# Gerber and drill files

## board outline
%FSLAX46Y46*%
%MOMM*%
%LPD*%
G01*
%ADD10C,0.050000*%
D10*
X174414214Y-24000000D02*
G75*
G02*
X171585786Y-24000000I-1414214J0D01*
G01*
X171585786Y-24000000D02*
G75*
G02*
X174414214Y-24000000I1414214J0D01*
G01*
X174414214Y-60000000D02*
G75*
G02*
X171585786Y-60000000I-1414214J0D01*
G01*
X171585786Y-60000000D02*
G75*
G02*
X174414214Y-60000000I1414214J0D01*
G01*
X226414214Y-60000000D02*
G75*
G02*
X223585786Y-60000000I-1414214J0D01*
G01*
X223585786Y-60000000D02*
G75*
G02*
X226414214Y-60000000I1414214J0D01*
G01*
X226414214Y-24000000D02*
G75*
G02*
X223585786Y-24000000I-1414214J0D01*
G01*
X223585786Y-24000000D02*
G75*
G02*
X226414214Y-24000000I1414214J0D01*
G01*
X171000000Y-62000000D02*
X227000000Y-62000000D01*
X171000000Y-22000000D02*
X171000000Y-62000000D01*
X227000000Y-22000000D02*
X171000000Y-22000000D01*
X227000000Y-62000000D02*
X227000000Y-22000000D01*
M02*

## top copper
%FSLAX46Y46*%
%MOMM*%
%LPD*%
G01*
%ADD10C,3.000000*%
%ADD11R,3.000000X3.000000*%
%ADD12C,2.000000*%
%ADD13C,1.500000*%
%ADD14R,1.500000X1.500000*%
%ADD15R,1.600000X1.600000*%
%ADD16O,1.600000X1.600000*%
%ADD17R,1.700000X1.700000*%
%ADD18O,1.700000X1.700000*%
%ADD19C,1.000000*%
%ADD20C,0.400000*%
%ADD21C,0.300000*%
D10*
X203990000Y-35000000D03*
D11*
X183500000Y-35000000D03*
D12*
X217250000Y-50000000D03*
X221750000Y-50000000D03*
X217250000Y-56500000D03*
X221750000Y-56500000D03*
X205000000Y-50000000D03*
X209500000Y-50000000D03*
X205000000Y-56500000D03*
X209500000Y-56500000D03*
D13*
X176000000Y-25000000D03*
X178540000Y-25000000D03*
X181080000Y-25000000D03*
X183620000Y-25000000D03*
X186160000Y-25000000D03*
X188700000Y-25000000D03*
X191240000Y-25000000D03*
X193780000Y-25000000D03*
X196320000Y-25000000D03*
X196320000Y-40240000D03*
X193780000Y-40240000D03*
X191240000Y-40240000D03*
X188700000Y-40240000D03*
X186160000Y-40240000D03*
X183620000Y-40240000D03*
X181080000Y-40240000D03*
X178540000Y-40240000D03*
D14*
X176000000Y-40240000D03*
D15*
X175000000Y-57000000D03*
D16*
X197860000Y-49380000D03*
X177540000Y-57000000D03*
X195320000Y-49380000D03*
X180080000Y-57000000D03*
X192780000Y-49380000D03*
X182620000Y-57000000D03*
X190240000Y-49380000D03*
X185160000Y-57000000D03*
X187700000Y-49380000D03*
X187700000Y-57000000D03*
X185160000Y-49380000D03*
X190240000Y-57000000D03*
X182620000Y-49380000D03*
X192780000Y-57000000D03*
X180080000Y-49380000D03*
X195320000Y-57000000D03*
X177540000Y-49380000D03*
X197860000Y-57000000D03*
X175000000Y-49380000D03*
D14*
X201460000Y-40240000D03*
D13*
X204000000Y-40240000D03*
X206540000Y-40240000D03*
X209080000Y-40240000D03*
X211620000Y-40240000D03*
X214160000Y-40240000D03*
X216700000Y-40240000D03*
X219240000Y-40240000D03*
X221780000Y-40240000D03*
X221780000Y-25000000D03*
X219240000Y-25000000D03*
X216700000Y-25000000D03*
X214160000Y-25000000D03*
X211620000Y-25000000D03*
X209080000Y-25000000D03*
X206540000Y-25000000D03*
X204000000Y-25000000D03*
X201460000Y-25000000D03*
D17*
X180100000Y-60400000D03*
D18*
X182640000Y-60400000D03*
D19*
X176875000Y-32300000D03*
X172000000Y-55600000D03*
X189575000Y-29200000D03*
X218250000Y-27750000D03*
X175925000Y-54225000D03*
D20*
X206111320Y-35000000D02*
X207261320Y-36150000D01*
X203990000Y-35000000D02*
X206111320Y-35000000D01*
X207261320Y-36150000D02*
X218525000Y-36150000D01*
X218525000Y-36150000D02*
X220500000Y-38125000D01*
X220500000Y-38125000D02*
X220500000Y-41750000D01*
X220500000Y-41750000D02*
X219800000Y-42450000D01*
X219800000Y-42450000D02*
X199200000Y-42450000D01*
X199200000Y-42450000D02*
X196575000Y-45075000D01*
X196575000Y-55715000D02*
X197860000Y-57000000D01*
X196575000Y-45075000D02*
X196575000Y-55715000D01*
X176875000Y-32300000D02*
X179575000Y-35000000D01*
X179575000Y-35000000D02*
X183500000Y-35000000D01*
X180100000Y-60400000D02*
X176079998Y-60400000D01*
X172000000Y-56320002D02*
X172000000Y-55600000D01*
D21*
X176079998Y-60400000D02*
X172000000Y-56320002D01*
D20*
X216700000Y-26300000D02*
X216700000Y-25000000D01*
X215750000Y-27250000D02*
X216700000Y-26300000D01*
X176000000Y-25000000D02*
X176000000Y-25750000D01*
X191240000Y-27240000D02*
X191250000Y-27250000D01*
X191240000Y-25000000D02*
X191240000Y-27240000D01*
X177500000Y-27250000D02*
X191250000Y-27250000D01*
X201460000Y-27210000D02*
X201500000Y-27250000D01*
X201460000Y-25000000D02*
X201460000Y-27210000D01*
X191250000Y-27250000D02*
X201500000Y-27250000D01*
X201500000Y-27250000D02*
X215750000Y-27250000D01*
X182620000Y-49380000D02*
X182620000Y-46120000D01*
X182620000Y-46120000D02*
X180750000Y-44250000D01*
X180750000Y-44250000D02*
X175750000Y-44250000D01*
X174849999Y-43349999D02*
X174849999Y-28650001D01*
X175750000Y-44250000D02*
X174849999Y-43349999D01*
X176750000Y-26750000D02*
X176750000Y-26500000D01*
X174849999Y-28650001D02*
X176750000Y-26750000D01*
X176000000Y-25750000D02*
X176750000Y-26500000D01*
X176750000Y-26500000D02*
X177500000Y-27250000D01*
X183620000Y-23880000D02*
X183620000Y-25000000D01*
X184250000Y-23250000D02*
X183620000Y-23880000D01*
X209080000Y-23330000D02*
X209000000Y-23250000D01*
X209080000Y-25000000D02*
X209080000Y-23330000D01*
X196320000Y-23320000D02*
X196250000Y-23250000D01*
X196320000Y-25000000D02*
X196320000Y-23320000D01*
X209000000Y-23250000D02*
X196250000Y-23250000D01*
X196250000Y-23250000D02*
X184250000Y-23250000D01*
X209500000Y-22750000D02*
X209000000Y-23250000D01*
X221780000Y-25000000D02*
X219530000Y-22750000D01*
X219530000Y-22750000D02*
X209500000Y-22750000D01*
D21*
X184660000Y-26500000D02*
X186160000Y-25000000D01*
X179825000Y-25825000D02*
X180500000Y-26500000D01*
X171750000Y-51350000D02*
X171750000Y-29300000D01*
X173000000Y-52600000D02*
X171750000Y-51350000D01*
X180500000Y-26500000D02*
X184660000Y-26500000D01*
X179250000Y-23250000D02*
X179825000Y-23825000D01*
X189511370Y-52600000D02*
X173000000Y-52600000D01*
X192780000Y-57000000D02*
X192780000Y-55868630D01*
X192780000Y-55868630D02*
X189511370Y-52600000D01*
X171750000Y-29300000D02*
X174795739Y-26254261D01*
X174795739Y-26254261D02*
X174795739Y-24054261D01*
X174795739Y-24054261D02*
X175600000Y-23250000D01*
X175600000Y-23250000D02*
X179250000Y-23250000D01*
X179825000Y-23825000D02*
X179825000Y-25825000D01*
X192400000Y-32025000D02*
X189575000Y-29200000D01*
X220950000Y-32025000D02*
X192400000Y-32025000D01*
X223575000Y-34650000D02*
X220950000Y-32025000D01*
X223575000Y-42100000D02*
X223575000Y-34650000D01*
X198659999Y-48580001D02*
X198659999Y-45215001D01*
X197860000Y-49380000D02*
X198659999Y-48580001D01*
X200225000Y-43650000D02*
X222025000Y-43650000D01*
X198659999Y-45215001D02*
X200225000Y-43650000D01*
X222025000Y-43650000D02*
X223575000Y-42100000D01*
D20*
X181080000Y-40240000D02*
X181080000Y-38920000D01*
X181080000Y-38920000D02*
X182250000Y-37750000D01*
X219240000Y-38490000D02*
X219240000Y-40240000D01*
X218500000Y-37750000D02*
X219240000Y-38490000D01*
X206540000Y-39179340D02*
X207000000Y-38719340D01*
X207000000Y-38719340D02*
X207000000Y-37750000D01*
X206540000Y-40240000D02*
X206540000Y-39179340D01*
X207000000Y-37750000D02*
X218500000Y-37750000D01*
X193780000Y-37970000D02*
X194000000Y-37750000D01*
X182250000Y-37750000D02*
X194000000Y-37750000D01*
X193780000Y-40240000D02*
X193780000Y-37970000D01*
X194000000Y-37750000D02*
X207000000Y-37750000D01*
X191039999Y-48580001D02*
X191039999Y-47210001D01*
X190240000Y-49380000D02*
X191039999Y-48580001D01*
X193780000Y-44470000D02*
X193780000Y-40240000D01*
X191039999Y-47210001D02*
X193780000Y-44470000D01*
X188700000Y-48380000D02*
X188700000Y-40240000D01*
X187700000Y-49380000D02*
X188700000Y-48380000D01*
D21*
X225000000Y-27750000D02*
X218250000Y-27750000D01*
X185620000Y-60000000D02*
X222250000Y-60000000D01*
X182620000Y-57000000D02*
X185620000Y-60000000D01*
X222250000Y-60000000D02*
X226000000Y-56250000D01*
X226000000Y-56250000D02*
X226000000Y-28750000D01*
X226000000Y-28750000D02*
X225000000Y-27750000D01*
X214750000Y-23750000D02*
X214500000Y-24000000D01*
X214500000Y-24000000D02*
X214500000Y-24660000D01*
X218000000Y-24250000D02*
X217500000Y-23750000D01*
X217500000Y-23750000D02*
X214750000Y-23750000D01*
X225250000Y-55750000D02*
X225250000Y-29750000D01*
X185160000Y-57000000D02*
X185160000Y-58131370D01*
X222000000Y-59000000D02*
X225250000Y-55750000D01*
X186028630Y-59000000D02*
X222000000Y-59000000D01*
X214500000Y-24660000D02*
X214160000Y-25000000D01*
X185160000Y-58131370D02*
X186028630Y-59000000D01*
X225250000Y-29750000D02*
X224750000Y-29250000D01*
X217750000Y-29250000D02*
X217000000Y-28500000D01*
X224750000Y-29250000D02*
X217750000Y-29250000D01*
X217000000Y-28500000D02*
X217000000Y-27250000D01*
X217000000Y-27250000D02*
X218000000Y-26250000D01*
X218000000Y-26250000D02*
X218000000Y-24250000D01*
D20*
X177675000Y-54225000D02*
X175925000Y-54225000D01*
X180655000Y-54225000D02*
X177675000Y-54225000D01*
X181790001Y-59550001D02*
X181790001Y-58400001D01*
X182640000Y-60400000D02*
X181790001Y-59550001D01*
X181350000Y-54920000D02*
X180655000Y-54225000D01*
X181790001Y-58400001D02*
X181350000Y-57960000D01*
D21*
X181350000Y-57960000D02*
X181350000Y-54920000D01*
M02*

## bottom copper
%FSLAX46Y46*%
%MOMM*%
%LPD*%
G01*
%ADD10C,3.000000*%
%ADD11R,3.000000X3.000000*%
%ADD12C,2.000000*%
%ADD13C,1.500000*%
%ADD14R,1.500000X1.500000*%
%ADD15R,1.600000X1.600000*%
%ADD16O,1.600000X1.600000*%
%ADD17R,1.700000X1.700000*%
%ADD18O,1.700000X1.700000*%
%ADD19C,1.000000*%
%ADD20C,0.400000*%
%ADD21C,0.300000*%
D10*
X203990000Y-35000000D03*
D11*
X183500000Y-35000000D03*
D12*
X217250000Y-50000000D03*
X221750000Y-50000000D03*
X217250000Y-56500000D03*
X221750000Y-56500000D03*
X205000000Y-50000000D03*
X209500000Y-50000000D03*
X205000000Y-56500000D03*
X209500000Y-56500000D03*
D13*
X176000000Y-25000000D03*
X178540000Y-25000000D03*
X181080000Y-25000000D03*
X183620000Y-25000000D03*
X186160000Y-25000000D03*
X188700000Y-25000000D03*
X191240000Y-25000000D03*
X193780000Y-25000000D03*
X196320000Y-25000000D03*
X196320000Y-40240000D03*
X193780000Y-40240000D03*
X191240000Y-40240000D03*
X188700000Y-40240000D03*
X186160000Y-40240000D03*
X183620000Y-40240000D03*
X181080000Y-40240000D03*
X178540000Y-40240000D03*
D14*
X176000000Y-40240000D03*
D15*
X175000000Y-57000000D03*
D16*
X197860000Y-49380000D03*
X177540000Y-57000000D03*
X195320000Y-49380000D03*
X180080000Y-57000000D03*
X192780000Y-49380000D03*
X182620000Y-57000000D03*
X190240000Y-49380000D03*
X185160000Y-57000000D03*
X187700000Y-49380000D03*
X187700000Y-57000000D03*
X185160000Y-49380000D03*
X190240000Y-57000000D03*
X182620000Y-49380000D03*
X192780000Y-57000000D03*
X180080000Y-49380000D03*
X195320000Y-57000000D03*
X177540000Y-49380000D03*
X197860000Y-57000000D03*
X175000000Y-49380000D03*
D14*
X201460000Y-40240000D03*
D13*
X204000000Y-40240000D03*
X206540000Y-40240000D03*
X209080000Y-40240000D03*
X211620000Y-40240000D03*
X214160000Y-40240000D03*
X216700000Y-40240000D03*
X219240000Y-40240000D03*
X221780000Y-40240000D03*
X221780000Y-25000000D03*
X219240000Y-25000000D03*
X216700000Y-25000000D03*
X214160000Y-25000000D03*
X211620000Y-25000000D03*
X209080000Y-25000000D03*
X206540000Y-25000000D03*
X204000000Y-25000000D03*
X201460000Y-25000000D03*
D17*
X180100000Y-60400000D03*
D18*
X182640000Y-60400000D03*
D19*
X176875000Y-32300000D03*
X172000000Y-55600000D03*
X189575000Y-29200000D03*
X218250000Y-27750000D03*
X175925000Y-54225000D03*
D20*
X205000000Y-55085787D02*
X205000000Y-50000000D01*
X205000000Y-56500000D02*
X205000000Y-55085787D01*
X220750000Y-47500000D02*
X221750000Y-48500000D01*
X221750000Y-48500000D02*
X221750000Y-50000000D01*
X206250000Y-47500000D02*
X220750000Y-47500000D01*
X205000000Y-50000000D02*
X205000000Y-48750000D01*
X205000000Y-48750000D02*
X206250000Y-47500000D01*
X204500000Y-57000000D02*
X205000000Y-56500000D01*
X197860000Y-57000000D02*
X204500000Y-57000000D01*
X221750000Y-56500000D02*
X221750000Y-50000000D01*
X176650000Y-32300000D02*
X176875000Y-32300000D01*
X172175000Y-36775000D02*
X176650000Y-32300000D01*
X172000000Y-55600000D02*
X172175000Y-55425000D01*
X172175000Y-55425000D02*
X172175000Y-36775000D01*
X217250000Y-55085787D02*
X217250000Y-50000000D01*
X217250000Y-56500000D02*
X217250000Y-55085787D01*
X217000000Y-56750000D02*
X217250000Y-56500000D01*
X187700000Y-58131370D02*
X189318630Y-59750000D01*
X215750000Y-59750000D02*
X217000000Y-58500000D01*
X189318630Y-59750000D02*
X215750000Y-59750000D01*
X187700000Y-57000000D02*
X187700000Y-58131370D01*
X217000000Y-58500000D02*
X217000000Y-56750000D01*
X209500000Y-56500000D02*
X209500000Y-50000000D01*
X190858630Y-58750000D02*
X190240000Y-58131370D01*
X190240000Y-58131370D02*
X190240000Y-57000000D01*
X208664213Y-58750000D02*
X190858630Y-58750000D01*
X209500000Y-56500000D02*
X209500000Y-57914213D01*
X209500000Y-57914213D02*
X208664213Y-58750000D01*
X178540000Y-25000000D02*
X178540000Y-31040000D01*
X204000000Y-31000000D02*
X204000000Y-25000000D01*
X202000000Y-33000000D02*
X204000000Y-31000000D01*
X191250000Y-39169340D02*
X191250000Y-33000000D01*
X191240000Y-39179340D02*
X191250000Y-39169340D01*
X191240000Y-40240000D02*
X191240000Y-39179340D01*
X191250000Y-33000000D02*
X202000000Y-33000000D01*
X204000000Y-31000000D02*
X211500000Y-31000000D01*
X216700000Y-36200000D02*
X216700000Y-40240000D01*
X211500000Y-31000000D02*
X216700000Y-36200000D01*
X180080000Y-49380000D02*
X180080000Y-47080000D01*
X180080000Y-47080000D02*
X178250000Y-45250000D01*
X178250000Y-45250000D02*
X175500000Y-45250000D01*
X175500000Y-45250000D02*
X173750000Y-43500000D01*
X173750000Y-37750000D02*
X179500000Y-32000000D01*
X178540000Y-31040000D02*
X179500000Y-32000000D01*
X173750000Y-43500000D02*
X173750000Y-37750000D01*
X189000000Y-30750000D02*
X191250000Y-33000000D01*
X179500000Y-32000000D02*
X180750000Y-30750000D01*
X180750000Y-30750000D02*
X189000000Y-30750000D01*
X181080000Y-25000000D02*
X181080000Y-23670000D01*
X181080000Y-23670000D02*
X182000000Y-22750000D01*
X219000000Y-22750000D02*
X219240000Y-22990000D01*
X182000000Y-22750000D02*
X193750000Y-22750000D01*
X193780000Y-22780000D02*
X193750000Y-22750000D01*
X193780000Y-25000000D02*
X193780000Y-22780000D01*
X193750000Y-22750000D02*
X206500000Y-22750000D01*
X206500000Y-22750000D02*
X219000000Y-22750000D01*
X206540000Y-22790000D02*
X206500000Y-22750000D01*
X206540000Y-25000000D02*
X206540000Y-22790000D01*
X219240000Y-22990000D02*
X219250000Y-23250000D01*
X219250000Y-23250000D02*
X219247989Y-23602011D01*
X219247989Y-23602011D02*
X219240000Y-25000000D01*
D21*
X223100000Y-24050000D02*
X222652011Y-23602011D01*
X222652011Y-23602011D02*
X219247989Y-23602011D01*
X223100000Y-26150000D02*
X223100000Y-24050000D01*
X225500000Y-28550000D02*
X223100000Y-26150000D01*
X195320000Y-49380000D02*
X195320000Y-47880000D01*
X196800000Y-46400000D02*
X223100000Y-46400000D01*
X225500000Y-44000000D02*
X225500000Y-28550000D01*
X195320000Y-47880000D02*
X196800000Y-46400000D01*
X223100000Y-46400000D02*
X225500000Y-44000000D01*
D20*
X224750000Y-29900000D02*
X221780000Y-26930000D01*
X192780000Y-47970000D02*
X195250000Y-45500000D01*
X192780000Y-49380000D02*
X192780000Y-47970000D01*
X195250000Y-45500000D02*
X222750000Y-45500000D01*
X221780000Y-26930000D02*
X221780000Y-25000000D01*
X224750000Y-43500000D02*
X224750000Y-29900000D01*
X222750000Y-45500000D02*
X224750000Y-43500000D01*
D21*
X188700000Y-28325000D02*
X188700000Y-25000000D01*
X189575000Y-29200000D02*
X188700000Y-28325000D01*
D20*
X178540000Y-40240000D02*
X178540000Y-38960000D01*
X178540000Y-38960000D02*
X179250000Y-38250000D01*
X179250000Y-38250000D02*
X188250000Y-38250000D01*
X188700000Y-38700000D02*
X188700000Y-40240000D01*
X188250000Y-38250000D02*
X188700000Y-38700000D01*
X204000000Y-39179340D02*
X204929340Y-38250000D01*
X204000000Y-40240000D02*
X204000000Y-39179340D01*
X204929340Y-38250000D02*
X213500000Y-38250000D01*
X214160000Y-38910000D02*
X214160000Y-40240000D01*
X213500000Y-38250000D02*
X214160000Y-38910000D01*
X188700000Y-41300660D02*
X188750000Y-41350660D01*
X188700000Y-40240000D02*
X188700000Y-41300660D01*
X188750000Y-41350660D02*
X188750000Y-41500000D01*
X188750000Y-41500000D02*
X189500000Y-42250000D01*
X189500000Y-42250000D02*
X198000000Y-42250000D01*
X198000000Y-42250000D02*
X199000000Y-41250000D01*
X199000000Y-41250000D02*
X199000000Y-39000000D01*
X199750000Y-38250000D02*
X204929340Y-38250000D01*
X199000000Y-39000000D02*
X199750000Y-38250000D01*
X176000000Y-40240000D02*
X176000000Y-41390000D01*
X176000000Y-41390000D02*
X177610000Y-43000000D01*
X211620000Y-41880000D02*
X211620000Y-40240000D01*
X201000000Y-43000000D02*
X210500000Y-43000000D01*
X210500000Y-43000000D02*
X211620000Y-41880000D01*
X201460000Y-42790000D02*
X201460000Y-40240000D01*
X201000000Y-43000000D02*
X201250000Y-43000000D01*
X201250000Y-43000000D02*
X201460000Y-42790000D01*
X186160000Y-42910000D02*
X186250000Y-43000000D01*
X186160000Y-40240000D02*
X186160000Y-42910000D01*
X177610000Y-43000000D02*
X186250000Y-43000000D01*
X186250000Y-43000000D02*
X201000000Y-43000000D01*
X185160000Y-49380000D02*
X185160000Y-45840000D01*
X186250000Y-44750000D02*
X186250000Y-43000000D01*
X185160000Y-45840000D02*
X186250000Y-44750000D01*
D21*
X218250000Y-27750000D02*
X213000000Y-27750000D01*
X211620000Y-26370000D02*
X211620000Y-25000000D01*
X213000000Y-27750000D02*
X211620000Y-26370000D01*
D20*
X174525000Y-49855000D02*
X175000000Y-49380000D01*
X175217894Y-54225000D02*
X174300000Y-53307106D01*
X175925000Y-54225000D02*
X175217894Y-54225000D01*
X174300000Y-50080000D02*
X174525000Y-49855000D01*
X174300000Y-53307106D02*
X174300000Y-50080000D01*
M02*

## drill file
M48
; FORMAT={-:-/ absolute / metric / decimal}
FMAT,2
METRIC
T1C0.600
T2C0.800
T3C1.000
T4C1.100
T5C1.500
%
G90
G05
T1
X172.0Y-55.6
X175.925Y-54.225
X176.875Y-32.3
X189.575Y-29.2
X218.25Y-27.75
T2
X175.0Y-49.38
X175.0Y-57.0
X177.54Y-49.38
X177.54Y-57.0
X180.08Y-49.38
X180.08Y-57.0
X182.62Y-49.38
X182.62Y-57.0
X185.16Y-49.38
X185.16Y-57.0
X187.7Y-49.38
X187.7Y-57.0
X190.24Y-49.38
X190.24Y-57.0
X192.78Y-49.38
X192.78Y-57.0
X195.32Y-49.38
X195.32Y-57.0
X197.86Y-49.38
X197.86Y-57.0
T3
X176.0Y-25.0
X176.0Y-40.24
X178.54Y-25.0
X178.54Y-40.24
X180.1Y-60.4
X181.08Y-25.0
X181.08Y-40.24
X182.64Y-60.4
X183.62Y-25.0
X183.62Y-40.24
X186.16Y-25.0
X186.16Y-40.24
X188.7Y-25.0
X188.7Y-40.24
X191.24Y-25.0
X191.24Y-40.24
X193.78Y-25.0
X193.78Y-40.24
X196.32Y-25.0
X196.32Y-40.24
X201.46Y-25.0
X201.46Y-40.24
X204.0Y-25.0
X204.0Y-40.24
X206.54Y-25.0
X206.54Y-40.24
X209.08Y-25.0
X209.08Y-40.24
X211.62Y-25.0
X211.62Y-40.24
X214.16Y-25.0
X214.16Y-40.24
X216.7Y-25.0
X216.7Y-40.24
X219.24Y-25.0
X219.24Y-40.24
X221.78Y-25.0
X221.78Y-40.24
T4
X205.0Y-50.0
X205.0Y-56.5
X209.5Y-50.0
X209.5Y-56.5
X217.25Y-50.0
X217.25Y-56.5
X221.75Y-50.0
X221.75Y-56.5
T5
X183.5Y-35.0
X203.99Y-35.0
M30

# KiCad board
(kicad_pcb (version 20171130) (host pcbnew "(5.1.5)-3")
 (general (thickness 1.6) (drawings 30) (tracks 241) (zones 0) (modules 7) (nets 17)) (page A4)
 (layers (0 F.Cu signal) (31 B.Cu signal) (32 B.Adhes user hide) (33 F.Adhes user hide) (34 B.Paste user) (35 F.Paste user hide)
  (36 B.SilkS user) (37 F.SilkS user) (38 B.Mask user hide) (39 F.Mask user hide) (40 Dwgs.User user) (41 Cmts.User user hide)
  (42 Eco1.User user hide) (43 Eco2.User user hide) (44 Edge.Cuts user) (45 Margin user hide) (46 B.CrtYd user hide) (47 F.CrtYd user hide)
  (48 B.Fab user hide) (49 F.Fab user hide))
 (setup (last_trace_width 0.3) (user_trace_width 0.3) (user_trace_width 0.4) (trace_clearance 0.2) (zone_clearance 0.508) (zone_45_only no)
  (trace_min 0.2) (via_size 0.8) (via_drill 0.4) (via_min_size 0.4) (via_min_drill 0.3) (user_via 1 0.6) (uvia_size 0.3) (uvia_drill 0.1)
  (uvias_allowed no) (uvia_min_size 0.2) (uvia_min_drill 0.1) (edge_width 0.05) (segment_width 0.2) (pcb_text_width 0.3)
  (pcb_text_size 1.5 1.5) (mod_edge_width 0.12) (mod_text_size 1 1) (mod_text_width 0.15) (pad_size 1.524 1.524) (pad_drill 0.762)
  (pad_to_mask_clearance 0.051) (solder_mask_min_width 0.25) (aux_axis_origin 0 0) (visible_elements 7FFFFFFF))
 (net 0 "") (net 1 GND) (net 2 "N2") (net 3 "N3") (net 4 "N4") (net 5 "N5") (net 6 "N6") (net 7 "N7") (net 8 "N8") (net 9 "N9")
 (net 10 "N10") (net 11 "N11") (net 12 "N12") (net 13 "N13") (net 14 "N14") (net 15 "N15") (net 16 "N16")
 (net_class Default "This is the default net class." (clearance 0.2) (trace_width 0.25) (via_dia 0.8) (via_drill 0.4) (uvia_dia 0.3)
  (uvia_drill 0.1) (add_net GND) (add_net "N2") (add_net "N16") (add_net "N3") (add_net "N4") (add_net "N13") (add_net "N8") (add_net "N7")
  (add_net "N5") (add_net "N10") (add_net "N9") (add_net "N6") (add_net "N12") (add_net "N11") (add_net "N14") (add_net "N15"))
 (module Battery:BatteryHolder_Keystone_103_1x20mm (layer B.Cu) (at 183.5 35)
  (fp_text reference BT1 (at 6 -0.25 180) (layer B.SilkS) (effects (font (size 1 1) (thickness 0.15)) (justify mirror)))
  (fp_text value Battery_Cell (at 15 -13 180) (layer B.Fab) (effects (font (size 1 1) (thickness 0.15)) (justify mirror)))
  (pad 2 thru_hole circle (at 20.49 0) (size 3 3) (drill 1.5) (layers *.Cu *.Mask) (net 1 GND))
  (pad 1 thru_hole rect (at 0 0) (size 3 3) (drill 1.5) (layers *.Cu *.Mask) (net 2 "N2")))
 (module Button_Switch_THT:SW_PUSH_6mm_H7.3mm (layer F.Cu) (at 217.25 56.5 90)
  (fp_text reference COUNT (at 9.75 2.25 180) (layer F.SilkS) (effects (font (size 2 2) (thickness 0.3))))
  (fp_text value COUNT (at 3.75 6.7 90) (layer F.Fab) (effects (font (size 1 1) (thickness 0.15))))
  (pad 1 thru_hole circle (at 6.5 0 180) (size 2 2) (drill 1.1) (layers *.Cu *.Mask) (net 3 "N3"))
  (pad 2 thru_hole circle (at 6.5 4.5 180) (size 2 2) (drill 1.1) (layers *.Cu *.Mask) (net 1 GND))
  (pad 1 thru_hole circle (at 0 0 180) (size 2 2) (drill 1.1) (layers *.Cu *.Mask) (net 3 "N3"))
  (pad 2 thru_hole circle (at 0 4.5 180) (size 2 2) (drill 1.1) (layers *.Cu *.Mask) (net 1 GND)))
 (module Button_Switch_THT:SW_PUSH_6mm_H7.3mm (layer F.Cu) (at 209.5 50 270)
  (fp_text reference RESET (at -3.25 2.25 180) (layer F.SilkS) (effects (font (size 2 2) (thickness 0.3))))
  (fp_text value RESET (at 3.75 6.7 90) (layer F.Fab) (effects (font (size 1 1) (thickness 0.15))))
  (pad 2 thru_hole circle (at 0 4.5) (size 2 2) (drill 1.1) (layers *.Cu *.Mask) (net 1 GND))
  (pad 1 thru_hole circle (at 0 0) (size 2 2) (drill 1.1) (layers *.Cu *.Mask) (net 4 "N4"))
  (pad 2 thru_hole circle (at 6.5 4.5) (size 2 2) (drill 1.1) (layers *.Cu *.Mask) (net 1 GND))
  (pad 1 thru_hole circle (at 6.5 0) (size 2 2) (drill 1.1) (layers *.Cu *.Mask) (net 4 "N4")))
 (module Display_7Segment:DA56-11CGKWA (layer F.Cu) (at 176 40.24 90)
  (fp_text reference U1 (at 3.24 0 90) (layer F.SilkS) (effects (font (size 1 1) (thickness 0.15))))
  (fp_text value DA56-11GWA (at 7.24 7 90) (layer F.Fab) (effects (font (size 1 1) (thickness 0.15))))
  (pad 18 thru_hole circle (at 15.24 0 90) (size 1.5 1.5) (drill 1) (layers *.Cu *.Mask) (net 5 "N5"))
  (pad 17 thru_hole circle (at 15.24 2.54 90) (size 1.5 1.5) (drill 1) (layers *.Cu *.Mask) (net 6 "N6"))
  (pad 16 thru_hole circle (at 15.24 5.08 90) (size 1.5 1.5) (drill 1) (layers *.Cu *.Mask) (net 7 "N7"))
  (pad 15 thru_hole circle (at 15.24 7.62 90) (size 1.5 1.5) (drill 1) (layers *.Cu *.Mask) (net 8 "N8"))
  (pad 14 thru_hole circle (at 15.24 10.16 90) (size 1.5 1.5) (drill 1) (layers *.Cu *.Mask) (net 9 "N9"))
  (pad 13 thru_hole circle (at 15.24 12.7 90) (size 1.5 1.5) (drill 1) (layers *.Cu *.Mask) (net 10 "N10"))
  (pad 12 thru_hole circle (at 15.24 15.24 90) (size 1.5 1.5) (drill 1) (layers *.Cu *.Mask) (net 5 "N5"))
  (pad 11 thru_hole circle (at 15.24 17.78 90) (size 1.5 1.5) (drill 1) (layers *.Cu *.Mask) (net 7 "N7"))
  (pad 10 thru_hole circle (at 15.24 20.32 90) (size 1.5 1.5) (drill 1) (layers *.Cu *.Mask) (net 8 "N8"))
  (pad 9 thru_hole circle (at 0 20.32 90) (size 1.5 1.5) (drill 1) (layers *.Cu *.Mask))
  (pad 8 thru_hole circle (at 0 17.78 90) (size 1.5 1.5) (drill 1) (layers *.Cu *.Mask) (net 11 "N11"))
  (pad 7 thru_hole circle (at 0 15.24 90) (size 1.5 1.5) (drill 1) (layers *.Cu *.Mask) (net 6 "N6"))
  (pad 6 thru_hole circle (at 0 12.7 90) (size 1.5 1.5) (drill 1) (layers *.Cu *.Mask) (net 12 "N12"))
  (pad 5 thru_hole circle (at 0 10.16 90) (size 1.5 1.5) (drill 1) (layers *.Cu *.Mask) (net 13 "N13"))
  (pad 4 thru_hole circle (at 0 7.62 90) (size 1.5 1.5) (drill 1) (layers *.Cu *.Mask))
  (pad 3 thru_hole circle (at 0 5.08 90) (size 1.5 1.5) (drill 1) (layers *.Cu *.Mask) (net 11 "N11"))
  (pad 2 thru_hole circle (at 0 2.54 90) (size 1.5 1.5) (drill 1) (layers *.Cu *.Mask) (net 12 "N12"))
  (pad 1 thru_hole rect (at 0 0 90) (size 1.5 1.5) (drill 1) (layers *.Cu *.Mask) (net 13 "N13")))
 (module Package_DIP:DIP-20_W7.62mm (layer F.Cu) (at 175 57 90)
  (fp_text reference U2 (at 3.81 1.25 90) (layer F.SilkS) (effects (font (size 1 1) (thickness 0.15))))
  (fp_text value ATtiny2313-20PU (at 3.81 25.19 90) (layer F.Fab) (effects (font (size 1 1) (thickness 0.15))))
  (pad 1 thru_hole rect (at 0 0 90) (size 1.6 1.6) (drill 0.8) (layers *.Cu *.Mask))
  (pad 11 thru_hole oval (at 7.62 22.86 90) (size 1.6 1.6) (drill 0.8) (layers *.Cu *.Mask) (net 10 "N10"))
  (pad 2 thru_hole oval (at 0 2.54 90) (size 1.6 1.6) (drill 0.8) (layers *.Cu *.Mask))
  (pad 12 thru_hole oval (at 7.62 20.32 90) (size 1.6 1.6) (drill 0.8) (layers *.Cu *.Mask) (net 7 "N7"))
  (pad 3 thru_hole oval (at 0 5.08 90) (size 1.6 1.6) (drill 0.8) (layers *.Cu *.Mask))
  (pad 13 thru_hole oval (at 7.62 17.78 90) (size 1.6 1.6) (drill 0.8) (layers *.Cu *.Mask) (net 8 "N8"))
  (pad 4 thru_hole oval (at 0 7.62 90) (size 1.6 1.6) (drill 0.8) (layers *.Cu *.Mask) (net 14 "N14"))
  (pad 14 thru_hole oval (at 7.62 15.24 90) (size 1.6 1.6) (drill 0.8) (layers *.Cu *.Mask) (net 11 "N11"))
  (pad 5 thru_hole oval (at 0 10.16 90) (size 1.6 1.6) (drill 0.8) (layers *.Cu *.Mask) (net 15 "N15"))
  (pad 15 thru_hole oval (at 7.62 12.7 90) (size 1.6 1.6) (drill 0.8) (layers *.Cu *.Mask) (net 12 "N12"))
  (pad 6 thru_hole oval (at 0 12.7 90) (size 1.6 1.6) (drill 0.8) (layers *.Cu *.Mask) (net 3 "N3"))
  (pad 16 thru_hole oval (at 7.62 10.16 90) (size 1.6 1.6) (drill 0.8) (layers *.Cu *.Mask) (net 13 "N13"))
  (pad 7 thru_hole oval (at 0 15.24 90) (size 1.6 1.6) (drill 0.8) (layers *.Cu *.Mask) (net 4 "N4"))
  (pad 17 thru_hole oval (at 7.62 7.62 90) (size 1.6 1.6) (drill 0.8) (layers *.Cu *.Mask) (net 5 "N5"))
  (pad 8 thru_hole oval (at 0 17.78 90) (size 1.6 1.6) (drill 0.8) (layers *.Cu *.Mask) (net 9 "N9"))
  (pad 18 thru_hole oval (at 7.62 5.08 90) (size 1.6 1.6) (drill 0.8) (layers *.Cu *.Mask) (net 6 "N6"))
  (pad 9 thru_hole oval (at 0 20.32 90) (size 1.6 1.6) (drill 0.8) (layers *.Cu *.Mask))
  (pad 19 thru_hole oval (at 7.62 2.54 90) (size 1.6 1.6) (drill 0.8) (layers *.Cu *.Mask))
  (pad 10 thru_hole oval (at 0 22.86 90) (size 1.6 1.6) (drill 0.8) (layers *.Cu *.Mask) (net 1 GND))
  (pad 20 thru_hole oval (at 7.62 0 90) (size 1.6 1.6) (drill 0.8) (layers *.Cu *.Mask) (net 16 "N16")))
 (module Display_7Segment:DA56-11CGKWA (layer F.Cu) (at 201.46 40.24 90)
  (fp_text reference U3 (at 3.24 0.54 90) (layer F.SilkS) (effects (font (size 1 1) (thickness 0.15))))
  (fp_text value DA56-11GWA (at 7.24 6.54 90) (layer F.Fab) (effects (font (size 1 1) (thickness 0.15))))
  (pad 1 thru_hole rect (at 0 0 90) (size 1.5 1.5) (drill 1) (layers *.Cu *.Mask) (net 13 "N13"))
  (pad 2 thru_hole circle (at 0 2.54 90) (size 1.5 1.5) (drill 1) (layers *.Cu *.Mask) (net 12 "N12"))
  (pad 3 thru_hole circle (at 0 5.08 90) (size 1.5 1.5) (drill 1) (layers *.Cu *.Mask) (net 11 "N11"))
  (pad 4 thru_hole circle (at 0 7.62 90) (size 1.5 1.5) (drill 1) (layers *.Cu *.Mask))
  (pad 5 thru_hole circle (at 0 10.16 90) (size 1.5 1.5) (drill 1) (layers *.Cu *.Mask) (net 13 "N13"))
  (pad 6 thru_hole circle (at 0 12.7 90) (size 1.5 1.5) (drill 1) (layers *.Cu *.Mask) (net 12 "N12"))
  (pad 7 thru_hole circle (at 0 15.24 90) (size 1.5 1.5) (drill 1) (layers *.Cu *.Mask) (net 6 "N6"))
  (pad 8 thru_hole circle (at 0 17.78 90) (size 1.5 1.5) (drill 1) (layers *.Cu *.Mask) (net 11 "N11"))
  (pad 9 thru_hole circle (at 0 20.32 90) (size 1.5 1.5) (drill 1) (layers *.Cu *.Mask))
  (pad 10 thru_hole circle (at 15.24 20.32 90) (size 1.5 1.5) (drill 1) (layers *.Cu *.Mask) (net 8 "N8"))
  (pad 11 thru_hole circle (at 15.24 17.78 90) (size 1.5 1.5) (drill 1) (layers *.Cu *.Mask) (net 7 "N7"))
  (pad 12 thru_hole circle (at 15.24 15.24 90) (size 1.5 1.5) (drill 1) (layers *.Cu *.Mask) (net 5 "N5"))
  (pad 13 thru_hole circle (at 15.24 12.7 90) (size 1.5 1.5) (drill 1) (layers *.Cu *.Mask) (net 15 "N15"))
  (pad 14 thru_hole circle (at 15.24 10.16 90) (size 1.5 1.5) (drill 1) (layers *.Cu *.Mask) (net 14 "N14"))
  (pad 15 thru_hole circle (at 15.24 7.62 90) (size 1.5 1.5) (drill 1) (layers *.Cu *.Mask) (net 8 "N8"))
  (pad 16 thru_hole circle (at 15.24 5.08 90) (size 1.5 1.5) (drill 1) (layers *.Cu *.Mask) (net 7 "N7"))
  (pad 17 thru_hole circle (at 15.24 2.54 90) (size 1.5 1.5) (drill 1) (layers *.Cu *.Mask) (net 6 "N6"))
  (pad 18 thru_hole circle (at 15.24 0 90) (size 1.5 1.5) (drill 1) (layers *.Cu *.Mask) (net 5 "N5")))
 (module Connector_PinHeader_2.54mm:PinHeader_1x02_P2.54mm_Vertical (layer F.Cu) (at 180.1 60.4 90)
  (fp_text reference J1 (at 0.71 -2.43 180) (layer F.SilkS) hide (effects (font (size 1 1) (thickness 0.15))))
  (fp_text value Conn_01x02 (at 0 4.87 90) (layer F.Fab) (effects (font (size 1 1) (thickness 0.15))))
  (pad 1 thru_hole rect (at 0 0 90) (size 1.7 1.7) (drill 1) (layers *.Cu *.Mask) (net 2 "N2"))
  (pad 2 thru_hole oval (at 0 2.54 90) (size 1.7 1.7) (drill 1) (layers *.Cu *.Mask) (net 16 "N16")))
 (gr_circle (center 173 24) (end 174 25) (layer Edge.Cuts) (width 0.05))
 (gr_circle (center 173 60) (end 174 61) (layer Edge.Cuts) (width 0.05))
 (gr_circle (center 225 60) (end 226 61) (layer Edge.Cuts) (width 0.05))
 (gr_circle (center 225 24) (end 226 25) (layer Edge.Cuts) (width 0.05))
 (gr_line (start 171 62) (end 227 62) (layer Edge.Cuts) (width 0.05))
 (gr_line (start 171 22) (end 171 62) (layer Edge.Cuts) (width 0.05))
 (gr_line (start 227 22) (end 171 22) (layer Edge.Cuts) (width 0.05))
 (gr_line (start 227 62) (end 227 22) (layer Edge.Cuts) (width 0.05))
 (segment (start 205 55.085787) (end 205 50) (width 0.4) (layer B.Cu) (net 1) (status 20))
 (segment (start 205 56.5) (end 205 55.085787) (width 0.4) (layer B.Cu) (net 1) (status 10))
 (segment (start 220.75 47.5) (end 221.75 48.5) (width 0.4) (layer B.Cu) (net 1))
 (segment (start 221.75 48.5) (end 221.75 50) (width 0.4) (layer B.Cu) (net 1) (status 20))
 (segment (start 206.25 47.5) (end 220.75 47.5) (width 0.4) (layer B.Cu) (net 1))
 (segment (start 205 50) (end 205 48.75) (width 0.4) (layer B.Cu) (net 1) (status 10))
 (segment (start 205 48.75) (end 206.25 47.5) (width 0.4) (layer B.Cu) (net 1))
 (segment (start 204.5 57) (end 205 56.5) (width 0.4) (layer B.Cu) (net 1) (status 30))
 (segment (start 197.86 57) (end 204.5 57) (width 0.4) (layer B.Cu) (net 1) (status 30))
 (segment (start 206.11132 35) (end 207.26132 36.15) (width 0.4) (layer F.Cu) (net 1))
 (segment (start 203.99 35) (end 206.11132 35) (width 0.4) (layer F.Cu) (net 1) (status 10))
 (segment (start 207.26132 36.15) (end 218.525 36.15) (width 0.4) (layer F.Cu) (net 1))
 (segment (start 218.525 36.15) (end 220.5 38.125) (width 0.4) (layer F.Cu) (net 1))
 (segment (start 220.5 38.125) (end 220.5 41.75) (width 0.4) (layer F.Cu) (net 1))
 (segment (start 220.5 41.75) (end 219.8 42.45) (width 0.4) (layer F.Cu) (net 1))
 (segment (start 219.8 42.45) (end 199.2 42.45) (width 0.4) (layer F.Cu) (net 1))
 (segment (start 199.2 42.45) (end 196.575 45.075) (width 0.4) (layer F.Cu) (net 1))
 (segment (start 196.575 55.715) (end 197.86 57) (width 0.4) (layer F.Cu) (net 1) (status 20))
 (segment (start 196.575 45.075) (end 196.575 55.715) (width 0.4) (layer F.Cu) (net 1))
 (segment (start 221.75 56.5) (end 221.75 50) (width 0.4) (layer B.Cu) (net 1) (status 30))
 (via (at 176.875 32.3) (size 1) (drill 0.6) (layers F.Cu B.Cu) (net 2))
 (segment (start 176.875 32.3) (end 179.575 35) (width 0.4) (layer F.Cu) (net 2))
 (segment (start 179.575 35) (end 183.5 35) (width 0.4) (layer F.Cu) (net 2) (status 20))
 (via (at 172 55.6) (size 1) (drill 0.6) (layers F.Cu B.Cu) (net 2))
 (segment (start 176.65 32.3) (end 176.875 32.3) (width 0.4) (layer B.Cu) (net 2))
 (segment (start 172.175 36.775) (end 176.65 32.3) (width 0.4) (layer B.Cu) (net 2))
 (segment (start 172 55.6) (end 172.175 55.425) (width 0.4) (layer B.Cu) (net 2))
 (segment (start 172.175 55.425) (end 172.175 36.775) (width 0.4) (layer B.Cu) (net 2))
 (segment (start 180.1 60.4) (end 176.079998 60.4) (width 0.4) (layer F.Cu) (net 2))
 (segment (start 172 56.320002) (end 172 55.6) (width 0.4) (layer F.Cu) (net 2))
 (segment (start 176.079998 60.4) (end 172 56.320002) (width 0.3) (layer F.Cu) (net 2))
 (segment (start 217.25 55.085787) (end 217.25 50) (width 0.4) (layer B.Cu) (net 3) (status 20))
 (segment (start 217.25 56.5) (end 217.25 55.085787) (width 0.4) (layer B.Cu) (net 3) (status 10))
 (segment (start 217 56.75) (end 217.25 56.5) (width 0.4) (layer B.Cu) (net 3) (status 30))
 (segment (start 187.7 58.13137) (end 189.31863 59.75) (width 0.4) (layer B.Cu) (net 3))
 (segment (start 215.75 59.75) (end 217 58.5) (width 0.4) (layer B.Cu) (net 3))
 (segment (start 189.31863 59.75) (end 215.75 59.75) (width 0.4) (layer B.Cu) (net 3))
 (segment (start 187.7 57) (end 187.7 58.13137) (width 0.4) (layer B.Cu) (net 3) (status 10))
 (segment (start 217 58.5) (end 217 56.75) (width 0.4) (layer B.Cu) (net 3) (status 20))
 (segment (start 209.5 56.5) (end 209.5 50) (width 0.4) (layer B.Cu) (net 4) (status 30))
 (segment (start 190.85863 58.75) (end 190.24 58.13137) (width 0.4) (layer B.Cu) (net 4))
 (segment (start 190.24 58.13137) (end 190.24 57) (width 0.4) (layer B.Cu) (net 4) (status 20))
 (segment (start 208.664213 58.75) (end 190.85863 58.75) (width 0.4) (layer B.Cu) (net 4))
 (segment (start 209.5 56.5) (end 209.5 57.914213) (width 0.4) (layer B.Cu) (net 4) (status 10))
 (segment (start 209.5 57.914213) (end 208.664213 58.75) (width 0.4) (layer B.Cu) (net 4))
 (segment (start 216.7 26.3) (end 216.7 25) (width 0.4) (layer F.Cu) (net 5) (status 20))
 (segment (start 215.75 27.25) (end 216.7 26.3) (width 0.4) (layer F.Cu) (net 5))
 (segment (start 176 25) (end 176 25.75) (width 0.4) (layer F.Cu) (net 5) (status 30))
 (segment (start 191.24 27.24) (end 191.25 27.25) (width 0.4) (layer F.Cu) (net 5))
 (segment (start 191.24 25) (end 191.24 27.24) (width 0.4) (layer F.Cu) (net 5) (status 10))
 (segment (start 177.5 27.25) (end 191.25 27.25) (width 0.4) (layer F.Cu) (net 5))
 (segment (start 201.46 27.21) (end 201.5 27.25) (width 0.4) (layer F.Cu) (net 5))
 (segment (start 201.46 25) (end 201.46 27.21) (width 0.4) (layer F.Cu) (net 5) (status 10))
 (segment (start 191.25 27.25) (end 201.5 27.25) (width 0.4) (layer F.Cu) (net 5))
 (segment (start 201.5 27.25) (end 215.75 27.25) (width 0.4) (layer F.Cu) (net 5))
 (segment (start 182.62 49.38) (end 182.62 46.12) (width 0.4) (layer F.Cu) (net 5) (status 10))
 (segment (start 182.62 46.12) (end 180.75 44.25) (width 0.4) (layer F.Cu) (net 5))
 (segment (start 180.75 44.25) (end 175.75 44.25) (width 0.4) (layer F.Cu) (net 5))
 (segment (start 174.849999 43.349999) (end 174.849999 28.650001) (width 0.4) (layer F.Cu) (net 5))
 (segment (start 175.75 44.25) (end 174.849999 43.349999) (width 0.4) (layer F.Cu) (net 5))
 (segment (start 176.75 26.75) (end 176.75 26.5) (width 0.4) (layer F.Cu) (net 5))
 (segment (start 174.849999 28.650001) (end 176.75 26.75) (width 0.4) (layer F.Cu) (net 5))
 (segment (start 176 25.75) (end 176.75 26.5) (width 0.4) (layer F.Cu) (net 5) (status 10))
 (segment (start 176.75 26.5) (end 177.5 27.25) (width 0.4) (layer F.Cu) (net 5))
 (segment (start 178.54 25) (end 178.54 31.04) (width 0.4) (layer B.Cu) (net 6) (status 10))
 (segment (start 204 31) (end 204 25) (width 0.4) (layer B.Cu) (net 6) (status 20))
 (segment (start 202 33) (end 204 31) (width 0.4) (layer B.Cu) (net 6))
 (segment (start 191.25 39.16934) (end 191.25 33) (width 0.4) (layer B.Cu) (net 6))
 (segment (start 191.24 39.17934) (end 191.25 39.16934) (width 0.4) (layer B.Cu) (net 6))
 (segment (start 191.24 40.24) (end 191.24 39.17934) (width 0.4) (layer B.Cu) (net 6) (status 10))
 (segment (start 191.25 33) (end 202 33) (width 0.4) (layer B.Cu) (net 6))
 (segment (start 204 31) (end 211.5 31) (width 0.4) (layer B.Cu) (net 6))
 (segment (start 216.7 36.2) (end 216.7 40.24) (width 0.4) (layer B.Cu) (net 6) (status 20))
 (segment (start 211.5 31) (end 216.7 36.2) (width 0.4) (layer B.Cu) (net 6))
 (segment (start 180.08 49.38) (end 180.08 47.08) (width 0.4) (layer B.Cu) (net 6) (status 10))
 (segment (start 180.08 47.08) (end 178.25 45.25) (width 0.4) (layer B.Cu) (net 6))
 (segment (start 178.25 45.25) (end 175.5 45.25) (width 0.4) (layer B.Cu) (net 6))
 (segment (start 175.5 45.25) (end 173.75 43.5) (width 0.4) (layer B.Cu) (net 6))
 (segment (start 173.75 37.75) (end 179.5 32) (width 0.4) (layer B.Cu) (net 6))
 (segment (start 178.54 31.04) (end 179.5 32) (width 0.4) (layer B.Cu) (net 6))
 (segment (start 173.75 43.5) (end 173.75 37.75) (width 0.4) (layer B.Cu) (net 6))
 (segment (start 189 30.75) (end 191.25 33) (width 0.4) (layer B.Cu) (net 6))
 (segment (start 179.5 32) (end 180.75 30.75) (width 0.4) (layer B.Cu) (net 6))
 (segment (start 180.75 30.75) (end 189 30.75) (width 0.4) (layer B.Cu) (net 6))
 (segment (start 181.08 25) (end 181.08 23.67) (width 0.4) (layer B.Cu) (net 7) (status 10))
 (segment (start 181.08 23.67) (end 182 22.75) (width 0.4) (layer B.Cu) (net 7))
 (segment (start 219 22.75) (end 219.24 22.99) (width 0.4) (layer B.Cu) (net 7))
 (segment (start 182 22.75) (end 193.75 22.75) (width 0.4) (layer B.Cu) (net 7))
 (segment (start 193.78 22.78) (end 193.75 22.75) (width 0.4) (layer B.Cu) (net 7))
 (segment (start 193.78 25) (end 193.78 22.78) (width 0.4) (layer B.Cu) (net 7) (status 10))
 (segment (start 193.75 22.75) (end 206.5 22.75) (width 0.4) (layer B.Cu) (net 7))
 (segment (start 206.5 22.75) (end 219 22.75) (width 0.4) (layer B.Cu) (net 7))
 (segment (start 206.54 22.79) (end 206.5 22.75) (width 0.4) (layer B.Cu) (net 7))
 (segment (start 206.54 25) (end 206.54 22.79) (width 0.4) (layer B.Cu) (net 7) (status 10))
 (segment (start 219.24 22.99) (end 219.25 23.25) (width 0.4) (layer B.Cu) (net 7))
 (segment (start 219.25 23.25) (end 219.247989 23.602011) (width 0.4) (layer B.Cu) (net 7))
 (segment (start 219.247989 23.602011) (end 219.24 25) (width 0.4) (layer B.Cu) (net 7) (status 20))
 (segment (start 223.1 24.05) (end 222.652011 23.602011) (width 0.3) (layer B.Cu) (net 7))
 (segment (start 222.652011 23.602011) (end 219.247989 23.602011) (width 0.3) (layer B.Cu) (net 7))
 (segment (start 223.1 26.15) (end 223.1 24.05) (width 0.3) (layer B.Cu) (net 7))
 (segment (start 225.5 28.55) (end 223.1 26.15) (width 0.3) (layer B.Cu) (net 7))
 (segment (start 195.32 49.38) (end 195.32 47.88) (width 0.3) (layer B.Cu) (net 7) (status 10))
 (segment (start 196.8 46.4) (end 223.1 46.4) (width 0.3) (layer B.Cu) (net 7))
 (segment (start 225.5 44) (end 225.5 28.55) (width 0.3) (layer B.Cu) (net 7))
 (segment (start 195.32 47.88) (end 196.8 46.4) (width 0.3) (layer B.Cu) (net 7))
 (segment (start 223.1 46.4) (end 225.5 44) (width 0.3) (layer B.Cu) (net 7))
 (segment (start 183.62 23.88) (end 183.62 25) (width 0.4) (layer F.Cu) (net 8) (status 20))
 (segment (start 184.25 23.25) (end 183.62 23.88) (width 0.4) (layer F.Cu) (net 8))
 (segment (start 209.08 23.33) (end 209 23.25) (width 0.4) (layer F.Cu) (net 8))
 (segment (start 209.08 25) (end 209.08 23.33) (width 0.4) (layer F.Cu) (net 8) (status 10))
 (segment (start 196.32 23.32) (end 196.25 23.25) (width 0.4) (layer F.Cu) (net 8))
 (segment (start 196.32 25) (end 196.32 23.32) (width 0.4) (layer F.Cu) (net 8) (status 10))
 (segment (start 209 23.25) (end 196.25 23.25) (width 0.4) (layer F.Cu) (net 8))
 (segment (start 196.25 23.25) (end 184.25 23.25) (width 0.4) (layer F.Cu) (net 8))
 (segment (start 209.5 22.75) (end 209 23.25) (width 0.4) (layer F.Cu) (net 8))
 (segment (start 221.78 25) (end 219.53 22.75) (width 0.4) (layer F.Cu) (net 8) (status 10))
 (segment (start 219.53 22.75) (end 209.5 22.75) (width 0.4) (layer F.Cu) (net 8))
 (segment (start 224.75 29.9) (end 221.78 26.93) (width 0.4) (layer B.Cu) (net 8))
 (segment (start 192.78 47.97) (end 195.25 45.5) (width 0.4) (layer B.Cu) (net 8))
 (segment (start 192.78 49.38) (end 192.78 47.97) (width 0.4) (layer B.Cu) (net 8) (status 10))
 (segment (start 195.25 45.5) (end 222.75 45.5) (width 0.4) (layer B.Cu) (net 8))
 (segment (start 221.78 26.93) (end 221.78 25) (width 0.4) (layer B.Cu) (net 8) (status 20))
 (segment (start 224.75 43.5) (end 224.75 29.9) (width 0.4) (layer B.Cu) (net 8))
 (segment (start 222.75 45.5) (end 224.75 43.5) (width 0.4) (layer B.Cu) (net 8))
 (segment (start 184.66 26.5) (end 186.16 25) (width 0.3) (layer F.Cu) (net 9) (status 20))
 (segment (start 179.825 25.825) (end 180.5 26.5) (width 0.3) (layer F.Cu) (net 9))
 (segment (start 171.75 51.35) (end 171.75 29.3) (width 0.3) (layer F.Cu) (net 9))
 (segment (start 173 52.6) (end 171.75 51.35) (width 0.3) (layer F.Cu) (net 9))
 (segment (start 180.5 26.5) (end 184.66 26.5) (width 0.3) (layer F.Cu) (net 9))
 (segment (start 179.25 23.25) (end 179.825 23.825) (width 0.3) (layer F.Cu) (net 9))
 (segment (start 189.51137 52.6) (end 173 52.6) (width 0.3) (layer F.Cu) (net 9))
 (segment (start 192.78 57) (end 192.78 55.86863) (width 0.3) (layer F.Cu) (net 9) (status 10))
 (segment (start 192.78 55.86863) (end 189.51137 52.6) (width 0.3) (layer F.Cu) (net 9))
 (segment (start 171.75 29.3) (end 174.795739 26.254261) (width 0.3) (layer F.Cu) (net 9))
 (segment (start 174.795739 26.254261) (end 174.795739 24.054261) (width 0.3) (layer F.Cu) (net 9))
 (segment (start 174.795739 24.054261) (end 175.6 23.25) (width 0.3) (layer F.Cu) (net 9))
 (segment (start 175.6 23.25) (end 179.25 23.25) (width 0.3) (layer F.Cu) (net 9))
 (segment (start 179.825 23.825) (end 179.825 25.825) (width 0.3) (layer F.Cu) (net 9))
 (via (at 189.575 29.2) (size 1) (drill 0.6) (layers F.Cu B.Cu) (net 10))
 (segment (start 188.7 28.325) (end 188.7 25) (width 0.3) (layer B.Cu) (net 10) (status 20))
 (segment (start 189.575 29.2) (end 188.7 28.325) (width 0.3) (layer B.Cu) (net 10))
 (segment (start 192.4 32.025) (end 189.575 29.2) (width 0.3) (layer F.Cu) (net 10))
 (segment (start 220.95 32.025) (end 192.4 32.025) (width 0.3) (layer F.Cu) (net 10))
 (segment (start 223.575 34.65) (end 220.95 32.025) (width 0.3) (layer F.Cu) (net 10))
 (segment (start 223.575 42.1) (end 223.575 34.65) (width 0.3) (layer F.Cu) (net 10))
 (segment (start 198.659999 48.580001) (end 198.659999 45.215001) (width 0.3) (layer F.Cu) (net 10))
 (segment (start 197.86 49.38) (end 198.659999 48.580001) (width 0.3) (layer F.Cu) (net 10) (status 10))
 (segment (start 200.225 43.65) (end 222.025 43.65) (width 0.3) (layer F.Cu) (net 10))
 (segment (start 198.659999 45.215001) (end 200.225 43.65) (width 0.3) (layer F.Cu) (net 10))
 (segment (start 222.025 43.65) (end 223.575 42.1) (width 0.3) (layer F.Cu) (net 10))
 (segment (start 181.08 40.24) (end 181.08 38.92) (width 0.4) (layer F.Cu) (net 11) (status 10))
 (segment (start 181.08 38.92) (end 182.25 37.75) (width 0.4) (layer F.Cu) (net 11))
 (segment (start 219.24 38.49) (end 219.24 40.24) (width 0.4) (layer F.Cu) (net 11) (status 20))
 (segment (start 218.5 37.75) (end 219.24 38.49) (width 0.4) (layer F.Cu) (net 11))
 (segment (start 206.54 39.17934) (end 207 38.71934) (width 0.4) (layer F.Cu) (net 11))
 (segment (start 207 38.71934) (end 207 37.75) (width 0.4) (layer F.Cu) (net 11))
 (segment (start 206.54 40.24) (end 206.54 39.17934) (width 0.4) (layer F.Cu) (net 11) (status 10))
 (segment (start 207 37.75) (end 218.5 37.75) (width 0.4) (layer F.Cu) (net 11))
 (segment (start 193.78 37.97) (end 194 37.75) (width 0.4) (layer F.Cu) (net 11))
 (segment (start 182.25 37.75) (end 194 37.75) (width 0.4) (layer F.Cu) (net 11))
 (segment (start 193.78 40.24) (end 193.78 37.97) (width 0.4) (layer F.Cu) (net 11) (status 10))
 (segment (start 194 37.75) (end 207 37.75) (width 0.4) (layer F.Cu) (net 11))
 (segment (start 191.039999 48.580001) (end 191.039999 47.210001) (width 0.4) (layer F.Cu) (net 11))
 (segment (start 190.24 49.38) (end 191.039999 48.580001) (width 0.4) (layer F.Cu) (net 11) (status 10))
 (segment (start 193.78 44.47) (end 193.78 40.24) (width 0.4) (layer F.Cu) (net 11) (status 20))
 (segment (start 191.039999 47.210001) (end 193.78 44.47) (width 0.4) (layer F.Cu) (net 11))
 (segment (start 178.54 40.24) (end 178.54 38.96) (width 0.4) (layer B.Cu) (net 12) (status 10))
 (segment (start 178.54 38.96) (end 179.25 38.25) (width 0.4) (layer B.Cu) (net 12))
 (segment (start 179.25 38.25) (end 188.25 38.25) (width 0.4) (layer B.Cu) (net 12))
 (segment (start 188.7 38.7) (end 188.7 40.24) (width 0.4) (layer B.Cu) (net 12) (status 20))
 (segment (start 188.25 38.25) (end 188.7 38.7) (width 0.4) (layer B.Cu) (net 12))
 (segment (start 204 39.17934) (end 204.92934 38.25) (width 0.4) (layer B.Cu) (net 12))
 (segment (start 204 40.24) (end 204 39.17934) (width 0.4) (layer B.Cu) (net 12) (status 10))
 (segment (start 204.92934 38.25) (end 213.5 38.25) (width 0.4) (layer B.Cu) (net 12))
 (segment (start 214.16 38.91) (end 214.16 40.24) (width 0.4) (layer B.Cu) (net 12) (status 20))
 (segment (start 213.5 38.25) (end 214.16 38.91) (width 0.4) (layer B.Cu) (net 12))
 (segment (start 188.7 41.30066) (end 188.75 41.35066) (width 0.4) (layer B.Cu) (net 12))
 (segment (start 188.7 40.24) (end 188.7 41.30066) (width 0.4) (layer B.Cu) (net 12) (status 10))
 (segment (start 188.75 41.35066) (end 188.75 41.5) (width 0.4) (layer B.Cu) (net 12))
 (segment (start 188.75 41.5) (end 189.5 42.25) (width 0.4) (layer B.Cu) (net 12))
 (segment (start 189.5 42.25) (end 198 42.25) (width 0.4) (layer B.Cu) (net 12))
 (segment (start 198 42.25) (end 199 41.25) (width 0.4) (layer B.Cu) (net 12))
 (segment (start 199 41.25) (end 199 39) (width 0.4) (layer B.Cu) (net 12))
 (segment (start 199.75 38.25) (end 204.92934 38.25) (width 0.4) (layer B.Cu) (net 12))
 (segment (start 199 39) (end 199.75 38.25) (width 0.4) (layer B.Cu) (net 12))
 (segment (start 188.7 48.38) (end 188.7 40.24) (width 0.4) (layer F.Cu) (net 12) (status 20))
 (segment (start 187.7 49.38) (end 188.7 48.38) (width 0.4) (layer F.Cu) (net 12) (status 10))
 (segment (start 176 40.24) (end 176 41.39) (width 0.4) (layer B.Cu) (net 13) (status 10))
 (segment (start 176 41.39) (end 177.61 43) (width 0.4) (layer B.Cu) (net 13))
 (segment (start 211.62 41.88) (end 211.62 40.24) (width 0.4) (layer B.Cu) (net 13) (status 20))
 (segment (start 201 43) (end 210.5 43) (width 0.4) (layer B.Cu) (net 13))
 (segment (start 210.5 43) (end 211.62 41.88) (width 0.4) (layer B.Cu) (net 13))
 (segment (start 201.46 42.79) (end 201.46 40.24) (width 0.4) (layer B.Cu) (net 13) (status 20))
 (segment (start 201 43) (end 201.25 43) (width 0.4) (layer B.Cu) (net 13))
 (segment (start 201.25 43) (end 201.46 42.79) (width 0.4) (layer B.Cu) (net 13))
 (segment (start 186.16 42.91) (end 186.25 43) (width 0.4) (layer B.Cu) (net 13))
 (segment (start 186.16 40.24) (end 186.16 42.91) (width 0.4) (layer B.Cu) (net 13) (status 10))
 (segment (start 177.61 43) (end 186.25 43) (width 0.4) (layer B.Cu) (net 13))
 (segment (start 186.25 43) (end 201 43) (width 0.4) (layer B.Cu) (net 13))
 (segment (start 185.16 49.38) (end 185.16 45.84) (width 0.4) (layer B.Cu) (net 13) (status 10))
 (segment (start 186.25 44.75) (end 186.25 43) (width 0.4) (layer B.Cu) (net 13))
 (segment (start 185.16 45.84) (end 186.25 44.75) (width 0.4) (layer B.Cu) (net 13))
 (via (at 218.25 27.75) (size 1) (drill 0.6) (layers F.Cu B.Cu) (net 14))
 (segment (start 218.25 27.75) (end 213 27.75) (width 0.3) (layer B.Cu) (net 14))
 (segment (start 211.62 26.37) (end 211.62 25) (width 0.3) (layer B.Cu) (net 14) (status 20))
 (segment (start 213 27.75) (end 211.62 26.37) (width 0.3) (layer B.Cu) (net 14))
 (segment (start 225 27.75) (end 218.25 27.75) (width 0.3) (layer F.Cu) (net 14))
 (segment (start 185.62 60) (end 222.25 60) (width 0.3) (layer F.Cu) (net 14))
 (segment (start 182.62 57) (end 185.62 60) (width 0.3) (layer F.Cu) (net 14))
 (segment (start 222.25 60) (end 226 56.25) (width 0.3) (layer F.Cu) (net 14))
 (segment (start 226 56.25) (end 226 28.75) (width 0.3) (layer F.Cu) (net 14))
 (segment (start 226 28.75) (end 225 27.75) (width 0.3) (layer F.Cu) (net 14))
 (segment (start 214.75 23.75) (end 214.5 24) (width 0.3) (layer F.Cu) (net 15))
 (segment (start 214.5 24) (end 214.5 24.66) (width 0.3) (layer F.Cu) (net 15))
 (segment (start 218 24.25) (end 217.5 23.75) (width 0.3) (layer F.Cu) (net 15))
 (segment (start 217.5 23.75) (end 214.75 23.75) (width 0.3) (layer F.Cu) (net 15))
 (segment (start 225.25 55.75) (end 225.25 29.75) (width 0.3) (layer F.Cu) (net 15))
 (segment (start 185.16 57) (end 185.16 58.13137) (width 0.3) (layer F.Cu) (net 15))
 (segment (start 222 59) (end 225.25 55.75) (width 0.3) (layer F.Cu) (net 15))
 (segment (start 186.02863 59) (end 222 59) (width 0.3) (layer F.Cu) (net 15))
 (segment (start 214.5 24.66) (end 214.16 25) (width 0.3) (layer F.Cu) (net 15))
 (segment (start 185.16 58.13137) (end 186.02863 59) (width 0.3) (layer F.Cu) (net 15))
 (segment (start 225.25 29.75) (end 224.75 29.25) (width 0.3) (layer F.Cu) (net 15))
 (segment (start 217.75 29.25) (end 217 28.5) (width 0.3) (layer F.Cu) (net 15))
 (segment (start 224.75 29.25) (end 217.75 29.25) (width 0.3) (layer F.Cu) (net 15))
 (segment (start 217 28.5) (end 217 27.25) (width 0.3) (layer F.Cu) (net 15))
 (segment (start 217 27.25) (end 218 26.25) (width 0.3) (layer F.Cu) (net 15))
 (segment (start 218 26.25) (end 218 24.25) (width 0.3) (layer F.Cu) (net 15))
 (via (at 175.925 54.225) (size 1) (drill 0.6) (layers F.Cu B.Cu) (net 16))
 (segment (start 174.525 49.855) (end 175 49.38) (width 0.4) (layer B.Cu) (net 16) (status 30))
 (segment (start 175.217894 54.225) (end 174.3 53.307106) (width 0.4) (layer B.Cu) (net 16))
 (segment (start 175.925 54.225) (end 175.217894 54.225) (width 0.4) (layer B.Cu) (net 16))
 (segment (start 174.3 50.08) (end 174.525 49.855) (width 0.4) (layer B.Cu) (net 16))
 (segment (start 174.3 53.307106) (end 174.3 50.08) (width 0.4) (layer B.Cu) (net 16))
 (segment (start 177.675 54.225) (end 175.925 54.225) (width 0.4) (layer F.Cu) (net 16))
 (segment (start 180.655 54.225) (end 177.675 54.225) (width 0.4) (layer F.Cu) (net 16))
 (segment (start 181.790001 59.550001) (end 181.790001 58.400001) (width 0.4) (layer F.Cu) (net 16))
 (segment (start 182.64 60.4) (end 181.790001 59.550001) (width 0.4) (layer F.Cu) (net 16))
 (segment (start 181.35 54.92) (end 180.655 54.225) (width 0.4) (layer F.Cu) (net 16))
 (segment (start 181.790001 58.400001) (end 181.35 57.96) (width 0.4) (layer F.Cu) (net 16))
 (segment (start 181.35 57.96) (end 181.35 54.92) (width 0.3) (layer F.Cu) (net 16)))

